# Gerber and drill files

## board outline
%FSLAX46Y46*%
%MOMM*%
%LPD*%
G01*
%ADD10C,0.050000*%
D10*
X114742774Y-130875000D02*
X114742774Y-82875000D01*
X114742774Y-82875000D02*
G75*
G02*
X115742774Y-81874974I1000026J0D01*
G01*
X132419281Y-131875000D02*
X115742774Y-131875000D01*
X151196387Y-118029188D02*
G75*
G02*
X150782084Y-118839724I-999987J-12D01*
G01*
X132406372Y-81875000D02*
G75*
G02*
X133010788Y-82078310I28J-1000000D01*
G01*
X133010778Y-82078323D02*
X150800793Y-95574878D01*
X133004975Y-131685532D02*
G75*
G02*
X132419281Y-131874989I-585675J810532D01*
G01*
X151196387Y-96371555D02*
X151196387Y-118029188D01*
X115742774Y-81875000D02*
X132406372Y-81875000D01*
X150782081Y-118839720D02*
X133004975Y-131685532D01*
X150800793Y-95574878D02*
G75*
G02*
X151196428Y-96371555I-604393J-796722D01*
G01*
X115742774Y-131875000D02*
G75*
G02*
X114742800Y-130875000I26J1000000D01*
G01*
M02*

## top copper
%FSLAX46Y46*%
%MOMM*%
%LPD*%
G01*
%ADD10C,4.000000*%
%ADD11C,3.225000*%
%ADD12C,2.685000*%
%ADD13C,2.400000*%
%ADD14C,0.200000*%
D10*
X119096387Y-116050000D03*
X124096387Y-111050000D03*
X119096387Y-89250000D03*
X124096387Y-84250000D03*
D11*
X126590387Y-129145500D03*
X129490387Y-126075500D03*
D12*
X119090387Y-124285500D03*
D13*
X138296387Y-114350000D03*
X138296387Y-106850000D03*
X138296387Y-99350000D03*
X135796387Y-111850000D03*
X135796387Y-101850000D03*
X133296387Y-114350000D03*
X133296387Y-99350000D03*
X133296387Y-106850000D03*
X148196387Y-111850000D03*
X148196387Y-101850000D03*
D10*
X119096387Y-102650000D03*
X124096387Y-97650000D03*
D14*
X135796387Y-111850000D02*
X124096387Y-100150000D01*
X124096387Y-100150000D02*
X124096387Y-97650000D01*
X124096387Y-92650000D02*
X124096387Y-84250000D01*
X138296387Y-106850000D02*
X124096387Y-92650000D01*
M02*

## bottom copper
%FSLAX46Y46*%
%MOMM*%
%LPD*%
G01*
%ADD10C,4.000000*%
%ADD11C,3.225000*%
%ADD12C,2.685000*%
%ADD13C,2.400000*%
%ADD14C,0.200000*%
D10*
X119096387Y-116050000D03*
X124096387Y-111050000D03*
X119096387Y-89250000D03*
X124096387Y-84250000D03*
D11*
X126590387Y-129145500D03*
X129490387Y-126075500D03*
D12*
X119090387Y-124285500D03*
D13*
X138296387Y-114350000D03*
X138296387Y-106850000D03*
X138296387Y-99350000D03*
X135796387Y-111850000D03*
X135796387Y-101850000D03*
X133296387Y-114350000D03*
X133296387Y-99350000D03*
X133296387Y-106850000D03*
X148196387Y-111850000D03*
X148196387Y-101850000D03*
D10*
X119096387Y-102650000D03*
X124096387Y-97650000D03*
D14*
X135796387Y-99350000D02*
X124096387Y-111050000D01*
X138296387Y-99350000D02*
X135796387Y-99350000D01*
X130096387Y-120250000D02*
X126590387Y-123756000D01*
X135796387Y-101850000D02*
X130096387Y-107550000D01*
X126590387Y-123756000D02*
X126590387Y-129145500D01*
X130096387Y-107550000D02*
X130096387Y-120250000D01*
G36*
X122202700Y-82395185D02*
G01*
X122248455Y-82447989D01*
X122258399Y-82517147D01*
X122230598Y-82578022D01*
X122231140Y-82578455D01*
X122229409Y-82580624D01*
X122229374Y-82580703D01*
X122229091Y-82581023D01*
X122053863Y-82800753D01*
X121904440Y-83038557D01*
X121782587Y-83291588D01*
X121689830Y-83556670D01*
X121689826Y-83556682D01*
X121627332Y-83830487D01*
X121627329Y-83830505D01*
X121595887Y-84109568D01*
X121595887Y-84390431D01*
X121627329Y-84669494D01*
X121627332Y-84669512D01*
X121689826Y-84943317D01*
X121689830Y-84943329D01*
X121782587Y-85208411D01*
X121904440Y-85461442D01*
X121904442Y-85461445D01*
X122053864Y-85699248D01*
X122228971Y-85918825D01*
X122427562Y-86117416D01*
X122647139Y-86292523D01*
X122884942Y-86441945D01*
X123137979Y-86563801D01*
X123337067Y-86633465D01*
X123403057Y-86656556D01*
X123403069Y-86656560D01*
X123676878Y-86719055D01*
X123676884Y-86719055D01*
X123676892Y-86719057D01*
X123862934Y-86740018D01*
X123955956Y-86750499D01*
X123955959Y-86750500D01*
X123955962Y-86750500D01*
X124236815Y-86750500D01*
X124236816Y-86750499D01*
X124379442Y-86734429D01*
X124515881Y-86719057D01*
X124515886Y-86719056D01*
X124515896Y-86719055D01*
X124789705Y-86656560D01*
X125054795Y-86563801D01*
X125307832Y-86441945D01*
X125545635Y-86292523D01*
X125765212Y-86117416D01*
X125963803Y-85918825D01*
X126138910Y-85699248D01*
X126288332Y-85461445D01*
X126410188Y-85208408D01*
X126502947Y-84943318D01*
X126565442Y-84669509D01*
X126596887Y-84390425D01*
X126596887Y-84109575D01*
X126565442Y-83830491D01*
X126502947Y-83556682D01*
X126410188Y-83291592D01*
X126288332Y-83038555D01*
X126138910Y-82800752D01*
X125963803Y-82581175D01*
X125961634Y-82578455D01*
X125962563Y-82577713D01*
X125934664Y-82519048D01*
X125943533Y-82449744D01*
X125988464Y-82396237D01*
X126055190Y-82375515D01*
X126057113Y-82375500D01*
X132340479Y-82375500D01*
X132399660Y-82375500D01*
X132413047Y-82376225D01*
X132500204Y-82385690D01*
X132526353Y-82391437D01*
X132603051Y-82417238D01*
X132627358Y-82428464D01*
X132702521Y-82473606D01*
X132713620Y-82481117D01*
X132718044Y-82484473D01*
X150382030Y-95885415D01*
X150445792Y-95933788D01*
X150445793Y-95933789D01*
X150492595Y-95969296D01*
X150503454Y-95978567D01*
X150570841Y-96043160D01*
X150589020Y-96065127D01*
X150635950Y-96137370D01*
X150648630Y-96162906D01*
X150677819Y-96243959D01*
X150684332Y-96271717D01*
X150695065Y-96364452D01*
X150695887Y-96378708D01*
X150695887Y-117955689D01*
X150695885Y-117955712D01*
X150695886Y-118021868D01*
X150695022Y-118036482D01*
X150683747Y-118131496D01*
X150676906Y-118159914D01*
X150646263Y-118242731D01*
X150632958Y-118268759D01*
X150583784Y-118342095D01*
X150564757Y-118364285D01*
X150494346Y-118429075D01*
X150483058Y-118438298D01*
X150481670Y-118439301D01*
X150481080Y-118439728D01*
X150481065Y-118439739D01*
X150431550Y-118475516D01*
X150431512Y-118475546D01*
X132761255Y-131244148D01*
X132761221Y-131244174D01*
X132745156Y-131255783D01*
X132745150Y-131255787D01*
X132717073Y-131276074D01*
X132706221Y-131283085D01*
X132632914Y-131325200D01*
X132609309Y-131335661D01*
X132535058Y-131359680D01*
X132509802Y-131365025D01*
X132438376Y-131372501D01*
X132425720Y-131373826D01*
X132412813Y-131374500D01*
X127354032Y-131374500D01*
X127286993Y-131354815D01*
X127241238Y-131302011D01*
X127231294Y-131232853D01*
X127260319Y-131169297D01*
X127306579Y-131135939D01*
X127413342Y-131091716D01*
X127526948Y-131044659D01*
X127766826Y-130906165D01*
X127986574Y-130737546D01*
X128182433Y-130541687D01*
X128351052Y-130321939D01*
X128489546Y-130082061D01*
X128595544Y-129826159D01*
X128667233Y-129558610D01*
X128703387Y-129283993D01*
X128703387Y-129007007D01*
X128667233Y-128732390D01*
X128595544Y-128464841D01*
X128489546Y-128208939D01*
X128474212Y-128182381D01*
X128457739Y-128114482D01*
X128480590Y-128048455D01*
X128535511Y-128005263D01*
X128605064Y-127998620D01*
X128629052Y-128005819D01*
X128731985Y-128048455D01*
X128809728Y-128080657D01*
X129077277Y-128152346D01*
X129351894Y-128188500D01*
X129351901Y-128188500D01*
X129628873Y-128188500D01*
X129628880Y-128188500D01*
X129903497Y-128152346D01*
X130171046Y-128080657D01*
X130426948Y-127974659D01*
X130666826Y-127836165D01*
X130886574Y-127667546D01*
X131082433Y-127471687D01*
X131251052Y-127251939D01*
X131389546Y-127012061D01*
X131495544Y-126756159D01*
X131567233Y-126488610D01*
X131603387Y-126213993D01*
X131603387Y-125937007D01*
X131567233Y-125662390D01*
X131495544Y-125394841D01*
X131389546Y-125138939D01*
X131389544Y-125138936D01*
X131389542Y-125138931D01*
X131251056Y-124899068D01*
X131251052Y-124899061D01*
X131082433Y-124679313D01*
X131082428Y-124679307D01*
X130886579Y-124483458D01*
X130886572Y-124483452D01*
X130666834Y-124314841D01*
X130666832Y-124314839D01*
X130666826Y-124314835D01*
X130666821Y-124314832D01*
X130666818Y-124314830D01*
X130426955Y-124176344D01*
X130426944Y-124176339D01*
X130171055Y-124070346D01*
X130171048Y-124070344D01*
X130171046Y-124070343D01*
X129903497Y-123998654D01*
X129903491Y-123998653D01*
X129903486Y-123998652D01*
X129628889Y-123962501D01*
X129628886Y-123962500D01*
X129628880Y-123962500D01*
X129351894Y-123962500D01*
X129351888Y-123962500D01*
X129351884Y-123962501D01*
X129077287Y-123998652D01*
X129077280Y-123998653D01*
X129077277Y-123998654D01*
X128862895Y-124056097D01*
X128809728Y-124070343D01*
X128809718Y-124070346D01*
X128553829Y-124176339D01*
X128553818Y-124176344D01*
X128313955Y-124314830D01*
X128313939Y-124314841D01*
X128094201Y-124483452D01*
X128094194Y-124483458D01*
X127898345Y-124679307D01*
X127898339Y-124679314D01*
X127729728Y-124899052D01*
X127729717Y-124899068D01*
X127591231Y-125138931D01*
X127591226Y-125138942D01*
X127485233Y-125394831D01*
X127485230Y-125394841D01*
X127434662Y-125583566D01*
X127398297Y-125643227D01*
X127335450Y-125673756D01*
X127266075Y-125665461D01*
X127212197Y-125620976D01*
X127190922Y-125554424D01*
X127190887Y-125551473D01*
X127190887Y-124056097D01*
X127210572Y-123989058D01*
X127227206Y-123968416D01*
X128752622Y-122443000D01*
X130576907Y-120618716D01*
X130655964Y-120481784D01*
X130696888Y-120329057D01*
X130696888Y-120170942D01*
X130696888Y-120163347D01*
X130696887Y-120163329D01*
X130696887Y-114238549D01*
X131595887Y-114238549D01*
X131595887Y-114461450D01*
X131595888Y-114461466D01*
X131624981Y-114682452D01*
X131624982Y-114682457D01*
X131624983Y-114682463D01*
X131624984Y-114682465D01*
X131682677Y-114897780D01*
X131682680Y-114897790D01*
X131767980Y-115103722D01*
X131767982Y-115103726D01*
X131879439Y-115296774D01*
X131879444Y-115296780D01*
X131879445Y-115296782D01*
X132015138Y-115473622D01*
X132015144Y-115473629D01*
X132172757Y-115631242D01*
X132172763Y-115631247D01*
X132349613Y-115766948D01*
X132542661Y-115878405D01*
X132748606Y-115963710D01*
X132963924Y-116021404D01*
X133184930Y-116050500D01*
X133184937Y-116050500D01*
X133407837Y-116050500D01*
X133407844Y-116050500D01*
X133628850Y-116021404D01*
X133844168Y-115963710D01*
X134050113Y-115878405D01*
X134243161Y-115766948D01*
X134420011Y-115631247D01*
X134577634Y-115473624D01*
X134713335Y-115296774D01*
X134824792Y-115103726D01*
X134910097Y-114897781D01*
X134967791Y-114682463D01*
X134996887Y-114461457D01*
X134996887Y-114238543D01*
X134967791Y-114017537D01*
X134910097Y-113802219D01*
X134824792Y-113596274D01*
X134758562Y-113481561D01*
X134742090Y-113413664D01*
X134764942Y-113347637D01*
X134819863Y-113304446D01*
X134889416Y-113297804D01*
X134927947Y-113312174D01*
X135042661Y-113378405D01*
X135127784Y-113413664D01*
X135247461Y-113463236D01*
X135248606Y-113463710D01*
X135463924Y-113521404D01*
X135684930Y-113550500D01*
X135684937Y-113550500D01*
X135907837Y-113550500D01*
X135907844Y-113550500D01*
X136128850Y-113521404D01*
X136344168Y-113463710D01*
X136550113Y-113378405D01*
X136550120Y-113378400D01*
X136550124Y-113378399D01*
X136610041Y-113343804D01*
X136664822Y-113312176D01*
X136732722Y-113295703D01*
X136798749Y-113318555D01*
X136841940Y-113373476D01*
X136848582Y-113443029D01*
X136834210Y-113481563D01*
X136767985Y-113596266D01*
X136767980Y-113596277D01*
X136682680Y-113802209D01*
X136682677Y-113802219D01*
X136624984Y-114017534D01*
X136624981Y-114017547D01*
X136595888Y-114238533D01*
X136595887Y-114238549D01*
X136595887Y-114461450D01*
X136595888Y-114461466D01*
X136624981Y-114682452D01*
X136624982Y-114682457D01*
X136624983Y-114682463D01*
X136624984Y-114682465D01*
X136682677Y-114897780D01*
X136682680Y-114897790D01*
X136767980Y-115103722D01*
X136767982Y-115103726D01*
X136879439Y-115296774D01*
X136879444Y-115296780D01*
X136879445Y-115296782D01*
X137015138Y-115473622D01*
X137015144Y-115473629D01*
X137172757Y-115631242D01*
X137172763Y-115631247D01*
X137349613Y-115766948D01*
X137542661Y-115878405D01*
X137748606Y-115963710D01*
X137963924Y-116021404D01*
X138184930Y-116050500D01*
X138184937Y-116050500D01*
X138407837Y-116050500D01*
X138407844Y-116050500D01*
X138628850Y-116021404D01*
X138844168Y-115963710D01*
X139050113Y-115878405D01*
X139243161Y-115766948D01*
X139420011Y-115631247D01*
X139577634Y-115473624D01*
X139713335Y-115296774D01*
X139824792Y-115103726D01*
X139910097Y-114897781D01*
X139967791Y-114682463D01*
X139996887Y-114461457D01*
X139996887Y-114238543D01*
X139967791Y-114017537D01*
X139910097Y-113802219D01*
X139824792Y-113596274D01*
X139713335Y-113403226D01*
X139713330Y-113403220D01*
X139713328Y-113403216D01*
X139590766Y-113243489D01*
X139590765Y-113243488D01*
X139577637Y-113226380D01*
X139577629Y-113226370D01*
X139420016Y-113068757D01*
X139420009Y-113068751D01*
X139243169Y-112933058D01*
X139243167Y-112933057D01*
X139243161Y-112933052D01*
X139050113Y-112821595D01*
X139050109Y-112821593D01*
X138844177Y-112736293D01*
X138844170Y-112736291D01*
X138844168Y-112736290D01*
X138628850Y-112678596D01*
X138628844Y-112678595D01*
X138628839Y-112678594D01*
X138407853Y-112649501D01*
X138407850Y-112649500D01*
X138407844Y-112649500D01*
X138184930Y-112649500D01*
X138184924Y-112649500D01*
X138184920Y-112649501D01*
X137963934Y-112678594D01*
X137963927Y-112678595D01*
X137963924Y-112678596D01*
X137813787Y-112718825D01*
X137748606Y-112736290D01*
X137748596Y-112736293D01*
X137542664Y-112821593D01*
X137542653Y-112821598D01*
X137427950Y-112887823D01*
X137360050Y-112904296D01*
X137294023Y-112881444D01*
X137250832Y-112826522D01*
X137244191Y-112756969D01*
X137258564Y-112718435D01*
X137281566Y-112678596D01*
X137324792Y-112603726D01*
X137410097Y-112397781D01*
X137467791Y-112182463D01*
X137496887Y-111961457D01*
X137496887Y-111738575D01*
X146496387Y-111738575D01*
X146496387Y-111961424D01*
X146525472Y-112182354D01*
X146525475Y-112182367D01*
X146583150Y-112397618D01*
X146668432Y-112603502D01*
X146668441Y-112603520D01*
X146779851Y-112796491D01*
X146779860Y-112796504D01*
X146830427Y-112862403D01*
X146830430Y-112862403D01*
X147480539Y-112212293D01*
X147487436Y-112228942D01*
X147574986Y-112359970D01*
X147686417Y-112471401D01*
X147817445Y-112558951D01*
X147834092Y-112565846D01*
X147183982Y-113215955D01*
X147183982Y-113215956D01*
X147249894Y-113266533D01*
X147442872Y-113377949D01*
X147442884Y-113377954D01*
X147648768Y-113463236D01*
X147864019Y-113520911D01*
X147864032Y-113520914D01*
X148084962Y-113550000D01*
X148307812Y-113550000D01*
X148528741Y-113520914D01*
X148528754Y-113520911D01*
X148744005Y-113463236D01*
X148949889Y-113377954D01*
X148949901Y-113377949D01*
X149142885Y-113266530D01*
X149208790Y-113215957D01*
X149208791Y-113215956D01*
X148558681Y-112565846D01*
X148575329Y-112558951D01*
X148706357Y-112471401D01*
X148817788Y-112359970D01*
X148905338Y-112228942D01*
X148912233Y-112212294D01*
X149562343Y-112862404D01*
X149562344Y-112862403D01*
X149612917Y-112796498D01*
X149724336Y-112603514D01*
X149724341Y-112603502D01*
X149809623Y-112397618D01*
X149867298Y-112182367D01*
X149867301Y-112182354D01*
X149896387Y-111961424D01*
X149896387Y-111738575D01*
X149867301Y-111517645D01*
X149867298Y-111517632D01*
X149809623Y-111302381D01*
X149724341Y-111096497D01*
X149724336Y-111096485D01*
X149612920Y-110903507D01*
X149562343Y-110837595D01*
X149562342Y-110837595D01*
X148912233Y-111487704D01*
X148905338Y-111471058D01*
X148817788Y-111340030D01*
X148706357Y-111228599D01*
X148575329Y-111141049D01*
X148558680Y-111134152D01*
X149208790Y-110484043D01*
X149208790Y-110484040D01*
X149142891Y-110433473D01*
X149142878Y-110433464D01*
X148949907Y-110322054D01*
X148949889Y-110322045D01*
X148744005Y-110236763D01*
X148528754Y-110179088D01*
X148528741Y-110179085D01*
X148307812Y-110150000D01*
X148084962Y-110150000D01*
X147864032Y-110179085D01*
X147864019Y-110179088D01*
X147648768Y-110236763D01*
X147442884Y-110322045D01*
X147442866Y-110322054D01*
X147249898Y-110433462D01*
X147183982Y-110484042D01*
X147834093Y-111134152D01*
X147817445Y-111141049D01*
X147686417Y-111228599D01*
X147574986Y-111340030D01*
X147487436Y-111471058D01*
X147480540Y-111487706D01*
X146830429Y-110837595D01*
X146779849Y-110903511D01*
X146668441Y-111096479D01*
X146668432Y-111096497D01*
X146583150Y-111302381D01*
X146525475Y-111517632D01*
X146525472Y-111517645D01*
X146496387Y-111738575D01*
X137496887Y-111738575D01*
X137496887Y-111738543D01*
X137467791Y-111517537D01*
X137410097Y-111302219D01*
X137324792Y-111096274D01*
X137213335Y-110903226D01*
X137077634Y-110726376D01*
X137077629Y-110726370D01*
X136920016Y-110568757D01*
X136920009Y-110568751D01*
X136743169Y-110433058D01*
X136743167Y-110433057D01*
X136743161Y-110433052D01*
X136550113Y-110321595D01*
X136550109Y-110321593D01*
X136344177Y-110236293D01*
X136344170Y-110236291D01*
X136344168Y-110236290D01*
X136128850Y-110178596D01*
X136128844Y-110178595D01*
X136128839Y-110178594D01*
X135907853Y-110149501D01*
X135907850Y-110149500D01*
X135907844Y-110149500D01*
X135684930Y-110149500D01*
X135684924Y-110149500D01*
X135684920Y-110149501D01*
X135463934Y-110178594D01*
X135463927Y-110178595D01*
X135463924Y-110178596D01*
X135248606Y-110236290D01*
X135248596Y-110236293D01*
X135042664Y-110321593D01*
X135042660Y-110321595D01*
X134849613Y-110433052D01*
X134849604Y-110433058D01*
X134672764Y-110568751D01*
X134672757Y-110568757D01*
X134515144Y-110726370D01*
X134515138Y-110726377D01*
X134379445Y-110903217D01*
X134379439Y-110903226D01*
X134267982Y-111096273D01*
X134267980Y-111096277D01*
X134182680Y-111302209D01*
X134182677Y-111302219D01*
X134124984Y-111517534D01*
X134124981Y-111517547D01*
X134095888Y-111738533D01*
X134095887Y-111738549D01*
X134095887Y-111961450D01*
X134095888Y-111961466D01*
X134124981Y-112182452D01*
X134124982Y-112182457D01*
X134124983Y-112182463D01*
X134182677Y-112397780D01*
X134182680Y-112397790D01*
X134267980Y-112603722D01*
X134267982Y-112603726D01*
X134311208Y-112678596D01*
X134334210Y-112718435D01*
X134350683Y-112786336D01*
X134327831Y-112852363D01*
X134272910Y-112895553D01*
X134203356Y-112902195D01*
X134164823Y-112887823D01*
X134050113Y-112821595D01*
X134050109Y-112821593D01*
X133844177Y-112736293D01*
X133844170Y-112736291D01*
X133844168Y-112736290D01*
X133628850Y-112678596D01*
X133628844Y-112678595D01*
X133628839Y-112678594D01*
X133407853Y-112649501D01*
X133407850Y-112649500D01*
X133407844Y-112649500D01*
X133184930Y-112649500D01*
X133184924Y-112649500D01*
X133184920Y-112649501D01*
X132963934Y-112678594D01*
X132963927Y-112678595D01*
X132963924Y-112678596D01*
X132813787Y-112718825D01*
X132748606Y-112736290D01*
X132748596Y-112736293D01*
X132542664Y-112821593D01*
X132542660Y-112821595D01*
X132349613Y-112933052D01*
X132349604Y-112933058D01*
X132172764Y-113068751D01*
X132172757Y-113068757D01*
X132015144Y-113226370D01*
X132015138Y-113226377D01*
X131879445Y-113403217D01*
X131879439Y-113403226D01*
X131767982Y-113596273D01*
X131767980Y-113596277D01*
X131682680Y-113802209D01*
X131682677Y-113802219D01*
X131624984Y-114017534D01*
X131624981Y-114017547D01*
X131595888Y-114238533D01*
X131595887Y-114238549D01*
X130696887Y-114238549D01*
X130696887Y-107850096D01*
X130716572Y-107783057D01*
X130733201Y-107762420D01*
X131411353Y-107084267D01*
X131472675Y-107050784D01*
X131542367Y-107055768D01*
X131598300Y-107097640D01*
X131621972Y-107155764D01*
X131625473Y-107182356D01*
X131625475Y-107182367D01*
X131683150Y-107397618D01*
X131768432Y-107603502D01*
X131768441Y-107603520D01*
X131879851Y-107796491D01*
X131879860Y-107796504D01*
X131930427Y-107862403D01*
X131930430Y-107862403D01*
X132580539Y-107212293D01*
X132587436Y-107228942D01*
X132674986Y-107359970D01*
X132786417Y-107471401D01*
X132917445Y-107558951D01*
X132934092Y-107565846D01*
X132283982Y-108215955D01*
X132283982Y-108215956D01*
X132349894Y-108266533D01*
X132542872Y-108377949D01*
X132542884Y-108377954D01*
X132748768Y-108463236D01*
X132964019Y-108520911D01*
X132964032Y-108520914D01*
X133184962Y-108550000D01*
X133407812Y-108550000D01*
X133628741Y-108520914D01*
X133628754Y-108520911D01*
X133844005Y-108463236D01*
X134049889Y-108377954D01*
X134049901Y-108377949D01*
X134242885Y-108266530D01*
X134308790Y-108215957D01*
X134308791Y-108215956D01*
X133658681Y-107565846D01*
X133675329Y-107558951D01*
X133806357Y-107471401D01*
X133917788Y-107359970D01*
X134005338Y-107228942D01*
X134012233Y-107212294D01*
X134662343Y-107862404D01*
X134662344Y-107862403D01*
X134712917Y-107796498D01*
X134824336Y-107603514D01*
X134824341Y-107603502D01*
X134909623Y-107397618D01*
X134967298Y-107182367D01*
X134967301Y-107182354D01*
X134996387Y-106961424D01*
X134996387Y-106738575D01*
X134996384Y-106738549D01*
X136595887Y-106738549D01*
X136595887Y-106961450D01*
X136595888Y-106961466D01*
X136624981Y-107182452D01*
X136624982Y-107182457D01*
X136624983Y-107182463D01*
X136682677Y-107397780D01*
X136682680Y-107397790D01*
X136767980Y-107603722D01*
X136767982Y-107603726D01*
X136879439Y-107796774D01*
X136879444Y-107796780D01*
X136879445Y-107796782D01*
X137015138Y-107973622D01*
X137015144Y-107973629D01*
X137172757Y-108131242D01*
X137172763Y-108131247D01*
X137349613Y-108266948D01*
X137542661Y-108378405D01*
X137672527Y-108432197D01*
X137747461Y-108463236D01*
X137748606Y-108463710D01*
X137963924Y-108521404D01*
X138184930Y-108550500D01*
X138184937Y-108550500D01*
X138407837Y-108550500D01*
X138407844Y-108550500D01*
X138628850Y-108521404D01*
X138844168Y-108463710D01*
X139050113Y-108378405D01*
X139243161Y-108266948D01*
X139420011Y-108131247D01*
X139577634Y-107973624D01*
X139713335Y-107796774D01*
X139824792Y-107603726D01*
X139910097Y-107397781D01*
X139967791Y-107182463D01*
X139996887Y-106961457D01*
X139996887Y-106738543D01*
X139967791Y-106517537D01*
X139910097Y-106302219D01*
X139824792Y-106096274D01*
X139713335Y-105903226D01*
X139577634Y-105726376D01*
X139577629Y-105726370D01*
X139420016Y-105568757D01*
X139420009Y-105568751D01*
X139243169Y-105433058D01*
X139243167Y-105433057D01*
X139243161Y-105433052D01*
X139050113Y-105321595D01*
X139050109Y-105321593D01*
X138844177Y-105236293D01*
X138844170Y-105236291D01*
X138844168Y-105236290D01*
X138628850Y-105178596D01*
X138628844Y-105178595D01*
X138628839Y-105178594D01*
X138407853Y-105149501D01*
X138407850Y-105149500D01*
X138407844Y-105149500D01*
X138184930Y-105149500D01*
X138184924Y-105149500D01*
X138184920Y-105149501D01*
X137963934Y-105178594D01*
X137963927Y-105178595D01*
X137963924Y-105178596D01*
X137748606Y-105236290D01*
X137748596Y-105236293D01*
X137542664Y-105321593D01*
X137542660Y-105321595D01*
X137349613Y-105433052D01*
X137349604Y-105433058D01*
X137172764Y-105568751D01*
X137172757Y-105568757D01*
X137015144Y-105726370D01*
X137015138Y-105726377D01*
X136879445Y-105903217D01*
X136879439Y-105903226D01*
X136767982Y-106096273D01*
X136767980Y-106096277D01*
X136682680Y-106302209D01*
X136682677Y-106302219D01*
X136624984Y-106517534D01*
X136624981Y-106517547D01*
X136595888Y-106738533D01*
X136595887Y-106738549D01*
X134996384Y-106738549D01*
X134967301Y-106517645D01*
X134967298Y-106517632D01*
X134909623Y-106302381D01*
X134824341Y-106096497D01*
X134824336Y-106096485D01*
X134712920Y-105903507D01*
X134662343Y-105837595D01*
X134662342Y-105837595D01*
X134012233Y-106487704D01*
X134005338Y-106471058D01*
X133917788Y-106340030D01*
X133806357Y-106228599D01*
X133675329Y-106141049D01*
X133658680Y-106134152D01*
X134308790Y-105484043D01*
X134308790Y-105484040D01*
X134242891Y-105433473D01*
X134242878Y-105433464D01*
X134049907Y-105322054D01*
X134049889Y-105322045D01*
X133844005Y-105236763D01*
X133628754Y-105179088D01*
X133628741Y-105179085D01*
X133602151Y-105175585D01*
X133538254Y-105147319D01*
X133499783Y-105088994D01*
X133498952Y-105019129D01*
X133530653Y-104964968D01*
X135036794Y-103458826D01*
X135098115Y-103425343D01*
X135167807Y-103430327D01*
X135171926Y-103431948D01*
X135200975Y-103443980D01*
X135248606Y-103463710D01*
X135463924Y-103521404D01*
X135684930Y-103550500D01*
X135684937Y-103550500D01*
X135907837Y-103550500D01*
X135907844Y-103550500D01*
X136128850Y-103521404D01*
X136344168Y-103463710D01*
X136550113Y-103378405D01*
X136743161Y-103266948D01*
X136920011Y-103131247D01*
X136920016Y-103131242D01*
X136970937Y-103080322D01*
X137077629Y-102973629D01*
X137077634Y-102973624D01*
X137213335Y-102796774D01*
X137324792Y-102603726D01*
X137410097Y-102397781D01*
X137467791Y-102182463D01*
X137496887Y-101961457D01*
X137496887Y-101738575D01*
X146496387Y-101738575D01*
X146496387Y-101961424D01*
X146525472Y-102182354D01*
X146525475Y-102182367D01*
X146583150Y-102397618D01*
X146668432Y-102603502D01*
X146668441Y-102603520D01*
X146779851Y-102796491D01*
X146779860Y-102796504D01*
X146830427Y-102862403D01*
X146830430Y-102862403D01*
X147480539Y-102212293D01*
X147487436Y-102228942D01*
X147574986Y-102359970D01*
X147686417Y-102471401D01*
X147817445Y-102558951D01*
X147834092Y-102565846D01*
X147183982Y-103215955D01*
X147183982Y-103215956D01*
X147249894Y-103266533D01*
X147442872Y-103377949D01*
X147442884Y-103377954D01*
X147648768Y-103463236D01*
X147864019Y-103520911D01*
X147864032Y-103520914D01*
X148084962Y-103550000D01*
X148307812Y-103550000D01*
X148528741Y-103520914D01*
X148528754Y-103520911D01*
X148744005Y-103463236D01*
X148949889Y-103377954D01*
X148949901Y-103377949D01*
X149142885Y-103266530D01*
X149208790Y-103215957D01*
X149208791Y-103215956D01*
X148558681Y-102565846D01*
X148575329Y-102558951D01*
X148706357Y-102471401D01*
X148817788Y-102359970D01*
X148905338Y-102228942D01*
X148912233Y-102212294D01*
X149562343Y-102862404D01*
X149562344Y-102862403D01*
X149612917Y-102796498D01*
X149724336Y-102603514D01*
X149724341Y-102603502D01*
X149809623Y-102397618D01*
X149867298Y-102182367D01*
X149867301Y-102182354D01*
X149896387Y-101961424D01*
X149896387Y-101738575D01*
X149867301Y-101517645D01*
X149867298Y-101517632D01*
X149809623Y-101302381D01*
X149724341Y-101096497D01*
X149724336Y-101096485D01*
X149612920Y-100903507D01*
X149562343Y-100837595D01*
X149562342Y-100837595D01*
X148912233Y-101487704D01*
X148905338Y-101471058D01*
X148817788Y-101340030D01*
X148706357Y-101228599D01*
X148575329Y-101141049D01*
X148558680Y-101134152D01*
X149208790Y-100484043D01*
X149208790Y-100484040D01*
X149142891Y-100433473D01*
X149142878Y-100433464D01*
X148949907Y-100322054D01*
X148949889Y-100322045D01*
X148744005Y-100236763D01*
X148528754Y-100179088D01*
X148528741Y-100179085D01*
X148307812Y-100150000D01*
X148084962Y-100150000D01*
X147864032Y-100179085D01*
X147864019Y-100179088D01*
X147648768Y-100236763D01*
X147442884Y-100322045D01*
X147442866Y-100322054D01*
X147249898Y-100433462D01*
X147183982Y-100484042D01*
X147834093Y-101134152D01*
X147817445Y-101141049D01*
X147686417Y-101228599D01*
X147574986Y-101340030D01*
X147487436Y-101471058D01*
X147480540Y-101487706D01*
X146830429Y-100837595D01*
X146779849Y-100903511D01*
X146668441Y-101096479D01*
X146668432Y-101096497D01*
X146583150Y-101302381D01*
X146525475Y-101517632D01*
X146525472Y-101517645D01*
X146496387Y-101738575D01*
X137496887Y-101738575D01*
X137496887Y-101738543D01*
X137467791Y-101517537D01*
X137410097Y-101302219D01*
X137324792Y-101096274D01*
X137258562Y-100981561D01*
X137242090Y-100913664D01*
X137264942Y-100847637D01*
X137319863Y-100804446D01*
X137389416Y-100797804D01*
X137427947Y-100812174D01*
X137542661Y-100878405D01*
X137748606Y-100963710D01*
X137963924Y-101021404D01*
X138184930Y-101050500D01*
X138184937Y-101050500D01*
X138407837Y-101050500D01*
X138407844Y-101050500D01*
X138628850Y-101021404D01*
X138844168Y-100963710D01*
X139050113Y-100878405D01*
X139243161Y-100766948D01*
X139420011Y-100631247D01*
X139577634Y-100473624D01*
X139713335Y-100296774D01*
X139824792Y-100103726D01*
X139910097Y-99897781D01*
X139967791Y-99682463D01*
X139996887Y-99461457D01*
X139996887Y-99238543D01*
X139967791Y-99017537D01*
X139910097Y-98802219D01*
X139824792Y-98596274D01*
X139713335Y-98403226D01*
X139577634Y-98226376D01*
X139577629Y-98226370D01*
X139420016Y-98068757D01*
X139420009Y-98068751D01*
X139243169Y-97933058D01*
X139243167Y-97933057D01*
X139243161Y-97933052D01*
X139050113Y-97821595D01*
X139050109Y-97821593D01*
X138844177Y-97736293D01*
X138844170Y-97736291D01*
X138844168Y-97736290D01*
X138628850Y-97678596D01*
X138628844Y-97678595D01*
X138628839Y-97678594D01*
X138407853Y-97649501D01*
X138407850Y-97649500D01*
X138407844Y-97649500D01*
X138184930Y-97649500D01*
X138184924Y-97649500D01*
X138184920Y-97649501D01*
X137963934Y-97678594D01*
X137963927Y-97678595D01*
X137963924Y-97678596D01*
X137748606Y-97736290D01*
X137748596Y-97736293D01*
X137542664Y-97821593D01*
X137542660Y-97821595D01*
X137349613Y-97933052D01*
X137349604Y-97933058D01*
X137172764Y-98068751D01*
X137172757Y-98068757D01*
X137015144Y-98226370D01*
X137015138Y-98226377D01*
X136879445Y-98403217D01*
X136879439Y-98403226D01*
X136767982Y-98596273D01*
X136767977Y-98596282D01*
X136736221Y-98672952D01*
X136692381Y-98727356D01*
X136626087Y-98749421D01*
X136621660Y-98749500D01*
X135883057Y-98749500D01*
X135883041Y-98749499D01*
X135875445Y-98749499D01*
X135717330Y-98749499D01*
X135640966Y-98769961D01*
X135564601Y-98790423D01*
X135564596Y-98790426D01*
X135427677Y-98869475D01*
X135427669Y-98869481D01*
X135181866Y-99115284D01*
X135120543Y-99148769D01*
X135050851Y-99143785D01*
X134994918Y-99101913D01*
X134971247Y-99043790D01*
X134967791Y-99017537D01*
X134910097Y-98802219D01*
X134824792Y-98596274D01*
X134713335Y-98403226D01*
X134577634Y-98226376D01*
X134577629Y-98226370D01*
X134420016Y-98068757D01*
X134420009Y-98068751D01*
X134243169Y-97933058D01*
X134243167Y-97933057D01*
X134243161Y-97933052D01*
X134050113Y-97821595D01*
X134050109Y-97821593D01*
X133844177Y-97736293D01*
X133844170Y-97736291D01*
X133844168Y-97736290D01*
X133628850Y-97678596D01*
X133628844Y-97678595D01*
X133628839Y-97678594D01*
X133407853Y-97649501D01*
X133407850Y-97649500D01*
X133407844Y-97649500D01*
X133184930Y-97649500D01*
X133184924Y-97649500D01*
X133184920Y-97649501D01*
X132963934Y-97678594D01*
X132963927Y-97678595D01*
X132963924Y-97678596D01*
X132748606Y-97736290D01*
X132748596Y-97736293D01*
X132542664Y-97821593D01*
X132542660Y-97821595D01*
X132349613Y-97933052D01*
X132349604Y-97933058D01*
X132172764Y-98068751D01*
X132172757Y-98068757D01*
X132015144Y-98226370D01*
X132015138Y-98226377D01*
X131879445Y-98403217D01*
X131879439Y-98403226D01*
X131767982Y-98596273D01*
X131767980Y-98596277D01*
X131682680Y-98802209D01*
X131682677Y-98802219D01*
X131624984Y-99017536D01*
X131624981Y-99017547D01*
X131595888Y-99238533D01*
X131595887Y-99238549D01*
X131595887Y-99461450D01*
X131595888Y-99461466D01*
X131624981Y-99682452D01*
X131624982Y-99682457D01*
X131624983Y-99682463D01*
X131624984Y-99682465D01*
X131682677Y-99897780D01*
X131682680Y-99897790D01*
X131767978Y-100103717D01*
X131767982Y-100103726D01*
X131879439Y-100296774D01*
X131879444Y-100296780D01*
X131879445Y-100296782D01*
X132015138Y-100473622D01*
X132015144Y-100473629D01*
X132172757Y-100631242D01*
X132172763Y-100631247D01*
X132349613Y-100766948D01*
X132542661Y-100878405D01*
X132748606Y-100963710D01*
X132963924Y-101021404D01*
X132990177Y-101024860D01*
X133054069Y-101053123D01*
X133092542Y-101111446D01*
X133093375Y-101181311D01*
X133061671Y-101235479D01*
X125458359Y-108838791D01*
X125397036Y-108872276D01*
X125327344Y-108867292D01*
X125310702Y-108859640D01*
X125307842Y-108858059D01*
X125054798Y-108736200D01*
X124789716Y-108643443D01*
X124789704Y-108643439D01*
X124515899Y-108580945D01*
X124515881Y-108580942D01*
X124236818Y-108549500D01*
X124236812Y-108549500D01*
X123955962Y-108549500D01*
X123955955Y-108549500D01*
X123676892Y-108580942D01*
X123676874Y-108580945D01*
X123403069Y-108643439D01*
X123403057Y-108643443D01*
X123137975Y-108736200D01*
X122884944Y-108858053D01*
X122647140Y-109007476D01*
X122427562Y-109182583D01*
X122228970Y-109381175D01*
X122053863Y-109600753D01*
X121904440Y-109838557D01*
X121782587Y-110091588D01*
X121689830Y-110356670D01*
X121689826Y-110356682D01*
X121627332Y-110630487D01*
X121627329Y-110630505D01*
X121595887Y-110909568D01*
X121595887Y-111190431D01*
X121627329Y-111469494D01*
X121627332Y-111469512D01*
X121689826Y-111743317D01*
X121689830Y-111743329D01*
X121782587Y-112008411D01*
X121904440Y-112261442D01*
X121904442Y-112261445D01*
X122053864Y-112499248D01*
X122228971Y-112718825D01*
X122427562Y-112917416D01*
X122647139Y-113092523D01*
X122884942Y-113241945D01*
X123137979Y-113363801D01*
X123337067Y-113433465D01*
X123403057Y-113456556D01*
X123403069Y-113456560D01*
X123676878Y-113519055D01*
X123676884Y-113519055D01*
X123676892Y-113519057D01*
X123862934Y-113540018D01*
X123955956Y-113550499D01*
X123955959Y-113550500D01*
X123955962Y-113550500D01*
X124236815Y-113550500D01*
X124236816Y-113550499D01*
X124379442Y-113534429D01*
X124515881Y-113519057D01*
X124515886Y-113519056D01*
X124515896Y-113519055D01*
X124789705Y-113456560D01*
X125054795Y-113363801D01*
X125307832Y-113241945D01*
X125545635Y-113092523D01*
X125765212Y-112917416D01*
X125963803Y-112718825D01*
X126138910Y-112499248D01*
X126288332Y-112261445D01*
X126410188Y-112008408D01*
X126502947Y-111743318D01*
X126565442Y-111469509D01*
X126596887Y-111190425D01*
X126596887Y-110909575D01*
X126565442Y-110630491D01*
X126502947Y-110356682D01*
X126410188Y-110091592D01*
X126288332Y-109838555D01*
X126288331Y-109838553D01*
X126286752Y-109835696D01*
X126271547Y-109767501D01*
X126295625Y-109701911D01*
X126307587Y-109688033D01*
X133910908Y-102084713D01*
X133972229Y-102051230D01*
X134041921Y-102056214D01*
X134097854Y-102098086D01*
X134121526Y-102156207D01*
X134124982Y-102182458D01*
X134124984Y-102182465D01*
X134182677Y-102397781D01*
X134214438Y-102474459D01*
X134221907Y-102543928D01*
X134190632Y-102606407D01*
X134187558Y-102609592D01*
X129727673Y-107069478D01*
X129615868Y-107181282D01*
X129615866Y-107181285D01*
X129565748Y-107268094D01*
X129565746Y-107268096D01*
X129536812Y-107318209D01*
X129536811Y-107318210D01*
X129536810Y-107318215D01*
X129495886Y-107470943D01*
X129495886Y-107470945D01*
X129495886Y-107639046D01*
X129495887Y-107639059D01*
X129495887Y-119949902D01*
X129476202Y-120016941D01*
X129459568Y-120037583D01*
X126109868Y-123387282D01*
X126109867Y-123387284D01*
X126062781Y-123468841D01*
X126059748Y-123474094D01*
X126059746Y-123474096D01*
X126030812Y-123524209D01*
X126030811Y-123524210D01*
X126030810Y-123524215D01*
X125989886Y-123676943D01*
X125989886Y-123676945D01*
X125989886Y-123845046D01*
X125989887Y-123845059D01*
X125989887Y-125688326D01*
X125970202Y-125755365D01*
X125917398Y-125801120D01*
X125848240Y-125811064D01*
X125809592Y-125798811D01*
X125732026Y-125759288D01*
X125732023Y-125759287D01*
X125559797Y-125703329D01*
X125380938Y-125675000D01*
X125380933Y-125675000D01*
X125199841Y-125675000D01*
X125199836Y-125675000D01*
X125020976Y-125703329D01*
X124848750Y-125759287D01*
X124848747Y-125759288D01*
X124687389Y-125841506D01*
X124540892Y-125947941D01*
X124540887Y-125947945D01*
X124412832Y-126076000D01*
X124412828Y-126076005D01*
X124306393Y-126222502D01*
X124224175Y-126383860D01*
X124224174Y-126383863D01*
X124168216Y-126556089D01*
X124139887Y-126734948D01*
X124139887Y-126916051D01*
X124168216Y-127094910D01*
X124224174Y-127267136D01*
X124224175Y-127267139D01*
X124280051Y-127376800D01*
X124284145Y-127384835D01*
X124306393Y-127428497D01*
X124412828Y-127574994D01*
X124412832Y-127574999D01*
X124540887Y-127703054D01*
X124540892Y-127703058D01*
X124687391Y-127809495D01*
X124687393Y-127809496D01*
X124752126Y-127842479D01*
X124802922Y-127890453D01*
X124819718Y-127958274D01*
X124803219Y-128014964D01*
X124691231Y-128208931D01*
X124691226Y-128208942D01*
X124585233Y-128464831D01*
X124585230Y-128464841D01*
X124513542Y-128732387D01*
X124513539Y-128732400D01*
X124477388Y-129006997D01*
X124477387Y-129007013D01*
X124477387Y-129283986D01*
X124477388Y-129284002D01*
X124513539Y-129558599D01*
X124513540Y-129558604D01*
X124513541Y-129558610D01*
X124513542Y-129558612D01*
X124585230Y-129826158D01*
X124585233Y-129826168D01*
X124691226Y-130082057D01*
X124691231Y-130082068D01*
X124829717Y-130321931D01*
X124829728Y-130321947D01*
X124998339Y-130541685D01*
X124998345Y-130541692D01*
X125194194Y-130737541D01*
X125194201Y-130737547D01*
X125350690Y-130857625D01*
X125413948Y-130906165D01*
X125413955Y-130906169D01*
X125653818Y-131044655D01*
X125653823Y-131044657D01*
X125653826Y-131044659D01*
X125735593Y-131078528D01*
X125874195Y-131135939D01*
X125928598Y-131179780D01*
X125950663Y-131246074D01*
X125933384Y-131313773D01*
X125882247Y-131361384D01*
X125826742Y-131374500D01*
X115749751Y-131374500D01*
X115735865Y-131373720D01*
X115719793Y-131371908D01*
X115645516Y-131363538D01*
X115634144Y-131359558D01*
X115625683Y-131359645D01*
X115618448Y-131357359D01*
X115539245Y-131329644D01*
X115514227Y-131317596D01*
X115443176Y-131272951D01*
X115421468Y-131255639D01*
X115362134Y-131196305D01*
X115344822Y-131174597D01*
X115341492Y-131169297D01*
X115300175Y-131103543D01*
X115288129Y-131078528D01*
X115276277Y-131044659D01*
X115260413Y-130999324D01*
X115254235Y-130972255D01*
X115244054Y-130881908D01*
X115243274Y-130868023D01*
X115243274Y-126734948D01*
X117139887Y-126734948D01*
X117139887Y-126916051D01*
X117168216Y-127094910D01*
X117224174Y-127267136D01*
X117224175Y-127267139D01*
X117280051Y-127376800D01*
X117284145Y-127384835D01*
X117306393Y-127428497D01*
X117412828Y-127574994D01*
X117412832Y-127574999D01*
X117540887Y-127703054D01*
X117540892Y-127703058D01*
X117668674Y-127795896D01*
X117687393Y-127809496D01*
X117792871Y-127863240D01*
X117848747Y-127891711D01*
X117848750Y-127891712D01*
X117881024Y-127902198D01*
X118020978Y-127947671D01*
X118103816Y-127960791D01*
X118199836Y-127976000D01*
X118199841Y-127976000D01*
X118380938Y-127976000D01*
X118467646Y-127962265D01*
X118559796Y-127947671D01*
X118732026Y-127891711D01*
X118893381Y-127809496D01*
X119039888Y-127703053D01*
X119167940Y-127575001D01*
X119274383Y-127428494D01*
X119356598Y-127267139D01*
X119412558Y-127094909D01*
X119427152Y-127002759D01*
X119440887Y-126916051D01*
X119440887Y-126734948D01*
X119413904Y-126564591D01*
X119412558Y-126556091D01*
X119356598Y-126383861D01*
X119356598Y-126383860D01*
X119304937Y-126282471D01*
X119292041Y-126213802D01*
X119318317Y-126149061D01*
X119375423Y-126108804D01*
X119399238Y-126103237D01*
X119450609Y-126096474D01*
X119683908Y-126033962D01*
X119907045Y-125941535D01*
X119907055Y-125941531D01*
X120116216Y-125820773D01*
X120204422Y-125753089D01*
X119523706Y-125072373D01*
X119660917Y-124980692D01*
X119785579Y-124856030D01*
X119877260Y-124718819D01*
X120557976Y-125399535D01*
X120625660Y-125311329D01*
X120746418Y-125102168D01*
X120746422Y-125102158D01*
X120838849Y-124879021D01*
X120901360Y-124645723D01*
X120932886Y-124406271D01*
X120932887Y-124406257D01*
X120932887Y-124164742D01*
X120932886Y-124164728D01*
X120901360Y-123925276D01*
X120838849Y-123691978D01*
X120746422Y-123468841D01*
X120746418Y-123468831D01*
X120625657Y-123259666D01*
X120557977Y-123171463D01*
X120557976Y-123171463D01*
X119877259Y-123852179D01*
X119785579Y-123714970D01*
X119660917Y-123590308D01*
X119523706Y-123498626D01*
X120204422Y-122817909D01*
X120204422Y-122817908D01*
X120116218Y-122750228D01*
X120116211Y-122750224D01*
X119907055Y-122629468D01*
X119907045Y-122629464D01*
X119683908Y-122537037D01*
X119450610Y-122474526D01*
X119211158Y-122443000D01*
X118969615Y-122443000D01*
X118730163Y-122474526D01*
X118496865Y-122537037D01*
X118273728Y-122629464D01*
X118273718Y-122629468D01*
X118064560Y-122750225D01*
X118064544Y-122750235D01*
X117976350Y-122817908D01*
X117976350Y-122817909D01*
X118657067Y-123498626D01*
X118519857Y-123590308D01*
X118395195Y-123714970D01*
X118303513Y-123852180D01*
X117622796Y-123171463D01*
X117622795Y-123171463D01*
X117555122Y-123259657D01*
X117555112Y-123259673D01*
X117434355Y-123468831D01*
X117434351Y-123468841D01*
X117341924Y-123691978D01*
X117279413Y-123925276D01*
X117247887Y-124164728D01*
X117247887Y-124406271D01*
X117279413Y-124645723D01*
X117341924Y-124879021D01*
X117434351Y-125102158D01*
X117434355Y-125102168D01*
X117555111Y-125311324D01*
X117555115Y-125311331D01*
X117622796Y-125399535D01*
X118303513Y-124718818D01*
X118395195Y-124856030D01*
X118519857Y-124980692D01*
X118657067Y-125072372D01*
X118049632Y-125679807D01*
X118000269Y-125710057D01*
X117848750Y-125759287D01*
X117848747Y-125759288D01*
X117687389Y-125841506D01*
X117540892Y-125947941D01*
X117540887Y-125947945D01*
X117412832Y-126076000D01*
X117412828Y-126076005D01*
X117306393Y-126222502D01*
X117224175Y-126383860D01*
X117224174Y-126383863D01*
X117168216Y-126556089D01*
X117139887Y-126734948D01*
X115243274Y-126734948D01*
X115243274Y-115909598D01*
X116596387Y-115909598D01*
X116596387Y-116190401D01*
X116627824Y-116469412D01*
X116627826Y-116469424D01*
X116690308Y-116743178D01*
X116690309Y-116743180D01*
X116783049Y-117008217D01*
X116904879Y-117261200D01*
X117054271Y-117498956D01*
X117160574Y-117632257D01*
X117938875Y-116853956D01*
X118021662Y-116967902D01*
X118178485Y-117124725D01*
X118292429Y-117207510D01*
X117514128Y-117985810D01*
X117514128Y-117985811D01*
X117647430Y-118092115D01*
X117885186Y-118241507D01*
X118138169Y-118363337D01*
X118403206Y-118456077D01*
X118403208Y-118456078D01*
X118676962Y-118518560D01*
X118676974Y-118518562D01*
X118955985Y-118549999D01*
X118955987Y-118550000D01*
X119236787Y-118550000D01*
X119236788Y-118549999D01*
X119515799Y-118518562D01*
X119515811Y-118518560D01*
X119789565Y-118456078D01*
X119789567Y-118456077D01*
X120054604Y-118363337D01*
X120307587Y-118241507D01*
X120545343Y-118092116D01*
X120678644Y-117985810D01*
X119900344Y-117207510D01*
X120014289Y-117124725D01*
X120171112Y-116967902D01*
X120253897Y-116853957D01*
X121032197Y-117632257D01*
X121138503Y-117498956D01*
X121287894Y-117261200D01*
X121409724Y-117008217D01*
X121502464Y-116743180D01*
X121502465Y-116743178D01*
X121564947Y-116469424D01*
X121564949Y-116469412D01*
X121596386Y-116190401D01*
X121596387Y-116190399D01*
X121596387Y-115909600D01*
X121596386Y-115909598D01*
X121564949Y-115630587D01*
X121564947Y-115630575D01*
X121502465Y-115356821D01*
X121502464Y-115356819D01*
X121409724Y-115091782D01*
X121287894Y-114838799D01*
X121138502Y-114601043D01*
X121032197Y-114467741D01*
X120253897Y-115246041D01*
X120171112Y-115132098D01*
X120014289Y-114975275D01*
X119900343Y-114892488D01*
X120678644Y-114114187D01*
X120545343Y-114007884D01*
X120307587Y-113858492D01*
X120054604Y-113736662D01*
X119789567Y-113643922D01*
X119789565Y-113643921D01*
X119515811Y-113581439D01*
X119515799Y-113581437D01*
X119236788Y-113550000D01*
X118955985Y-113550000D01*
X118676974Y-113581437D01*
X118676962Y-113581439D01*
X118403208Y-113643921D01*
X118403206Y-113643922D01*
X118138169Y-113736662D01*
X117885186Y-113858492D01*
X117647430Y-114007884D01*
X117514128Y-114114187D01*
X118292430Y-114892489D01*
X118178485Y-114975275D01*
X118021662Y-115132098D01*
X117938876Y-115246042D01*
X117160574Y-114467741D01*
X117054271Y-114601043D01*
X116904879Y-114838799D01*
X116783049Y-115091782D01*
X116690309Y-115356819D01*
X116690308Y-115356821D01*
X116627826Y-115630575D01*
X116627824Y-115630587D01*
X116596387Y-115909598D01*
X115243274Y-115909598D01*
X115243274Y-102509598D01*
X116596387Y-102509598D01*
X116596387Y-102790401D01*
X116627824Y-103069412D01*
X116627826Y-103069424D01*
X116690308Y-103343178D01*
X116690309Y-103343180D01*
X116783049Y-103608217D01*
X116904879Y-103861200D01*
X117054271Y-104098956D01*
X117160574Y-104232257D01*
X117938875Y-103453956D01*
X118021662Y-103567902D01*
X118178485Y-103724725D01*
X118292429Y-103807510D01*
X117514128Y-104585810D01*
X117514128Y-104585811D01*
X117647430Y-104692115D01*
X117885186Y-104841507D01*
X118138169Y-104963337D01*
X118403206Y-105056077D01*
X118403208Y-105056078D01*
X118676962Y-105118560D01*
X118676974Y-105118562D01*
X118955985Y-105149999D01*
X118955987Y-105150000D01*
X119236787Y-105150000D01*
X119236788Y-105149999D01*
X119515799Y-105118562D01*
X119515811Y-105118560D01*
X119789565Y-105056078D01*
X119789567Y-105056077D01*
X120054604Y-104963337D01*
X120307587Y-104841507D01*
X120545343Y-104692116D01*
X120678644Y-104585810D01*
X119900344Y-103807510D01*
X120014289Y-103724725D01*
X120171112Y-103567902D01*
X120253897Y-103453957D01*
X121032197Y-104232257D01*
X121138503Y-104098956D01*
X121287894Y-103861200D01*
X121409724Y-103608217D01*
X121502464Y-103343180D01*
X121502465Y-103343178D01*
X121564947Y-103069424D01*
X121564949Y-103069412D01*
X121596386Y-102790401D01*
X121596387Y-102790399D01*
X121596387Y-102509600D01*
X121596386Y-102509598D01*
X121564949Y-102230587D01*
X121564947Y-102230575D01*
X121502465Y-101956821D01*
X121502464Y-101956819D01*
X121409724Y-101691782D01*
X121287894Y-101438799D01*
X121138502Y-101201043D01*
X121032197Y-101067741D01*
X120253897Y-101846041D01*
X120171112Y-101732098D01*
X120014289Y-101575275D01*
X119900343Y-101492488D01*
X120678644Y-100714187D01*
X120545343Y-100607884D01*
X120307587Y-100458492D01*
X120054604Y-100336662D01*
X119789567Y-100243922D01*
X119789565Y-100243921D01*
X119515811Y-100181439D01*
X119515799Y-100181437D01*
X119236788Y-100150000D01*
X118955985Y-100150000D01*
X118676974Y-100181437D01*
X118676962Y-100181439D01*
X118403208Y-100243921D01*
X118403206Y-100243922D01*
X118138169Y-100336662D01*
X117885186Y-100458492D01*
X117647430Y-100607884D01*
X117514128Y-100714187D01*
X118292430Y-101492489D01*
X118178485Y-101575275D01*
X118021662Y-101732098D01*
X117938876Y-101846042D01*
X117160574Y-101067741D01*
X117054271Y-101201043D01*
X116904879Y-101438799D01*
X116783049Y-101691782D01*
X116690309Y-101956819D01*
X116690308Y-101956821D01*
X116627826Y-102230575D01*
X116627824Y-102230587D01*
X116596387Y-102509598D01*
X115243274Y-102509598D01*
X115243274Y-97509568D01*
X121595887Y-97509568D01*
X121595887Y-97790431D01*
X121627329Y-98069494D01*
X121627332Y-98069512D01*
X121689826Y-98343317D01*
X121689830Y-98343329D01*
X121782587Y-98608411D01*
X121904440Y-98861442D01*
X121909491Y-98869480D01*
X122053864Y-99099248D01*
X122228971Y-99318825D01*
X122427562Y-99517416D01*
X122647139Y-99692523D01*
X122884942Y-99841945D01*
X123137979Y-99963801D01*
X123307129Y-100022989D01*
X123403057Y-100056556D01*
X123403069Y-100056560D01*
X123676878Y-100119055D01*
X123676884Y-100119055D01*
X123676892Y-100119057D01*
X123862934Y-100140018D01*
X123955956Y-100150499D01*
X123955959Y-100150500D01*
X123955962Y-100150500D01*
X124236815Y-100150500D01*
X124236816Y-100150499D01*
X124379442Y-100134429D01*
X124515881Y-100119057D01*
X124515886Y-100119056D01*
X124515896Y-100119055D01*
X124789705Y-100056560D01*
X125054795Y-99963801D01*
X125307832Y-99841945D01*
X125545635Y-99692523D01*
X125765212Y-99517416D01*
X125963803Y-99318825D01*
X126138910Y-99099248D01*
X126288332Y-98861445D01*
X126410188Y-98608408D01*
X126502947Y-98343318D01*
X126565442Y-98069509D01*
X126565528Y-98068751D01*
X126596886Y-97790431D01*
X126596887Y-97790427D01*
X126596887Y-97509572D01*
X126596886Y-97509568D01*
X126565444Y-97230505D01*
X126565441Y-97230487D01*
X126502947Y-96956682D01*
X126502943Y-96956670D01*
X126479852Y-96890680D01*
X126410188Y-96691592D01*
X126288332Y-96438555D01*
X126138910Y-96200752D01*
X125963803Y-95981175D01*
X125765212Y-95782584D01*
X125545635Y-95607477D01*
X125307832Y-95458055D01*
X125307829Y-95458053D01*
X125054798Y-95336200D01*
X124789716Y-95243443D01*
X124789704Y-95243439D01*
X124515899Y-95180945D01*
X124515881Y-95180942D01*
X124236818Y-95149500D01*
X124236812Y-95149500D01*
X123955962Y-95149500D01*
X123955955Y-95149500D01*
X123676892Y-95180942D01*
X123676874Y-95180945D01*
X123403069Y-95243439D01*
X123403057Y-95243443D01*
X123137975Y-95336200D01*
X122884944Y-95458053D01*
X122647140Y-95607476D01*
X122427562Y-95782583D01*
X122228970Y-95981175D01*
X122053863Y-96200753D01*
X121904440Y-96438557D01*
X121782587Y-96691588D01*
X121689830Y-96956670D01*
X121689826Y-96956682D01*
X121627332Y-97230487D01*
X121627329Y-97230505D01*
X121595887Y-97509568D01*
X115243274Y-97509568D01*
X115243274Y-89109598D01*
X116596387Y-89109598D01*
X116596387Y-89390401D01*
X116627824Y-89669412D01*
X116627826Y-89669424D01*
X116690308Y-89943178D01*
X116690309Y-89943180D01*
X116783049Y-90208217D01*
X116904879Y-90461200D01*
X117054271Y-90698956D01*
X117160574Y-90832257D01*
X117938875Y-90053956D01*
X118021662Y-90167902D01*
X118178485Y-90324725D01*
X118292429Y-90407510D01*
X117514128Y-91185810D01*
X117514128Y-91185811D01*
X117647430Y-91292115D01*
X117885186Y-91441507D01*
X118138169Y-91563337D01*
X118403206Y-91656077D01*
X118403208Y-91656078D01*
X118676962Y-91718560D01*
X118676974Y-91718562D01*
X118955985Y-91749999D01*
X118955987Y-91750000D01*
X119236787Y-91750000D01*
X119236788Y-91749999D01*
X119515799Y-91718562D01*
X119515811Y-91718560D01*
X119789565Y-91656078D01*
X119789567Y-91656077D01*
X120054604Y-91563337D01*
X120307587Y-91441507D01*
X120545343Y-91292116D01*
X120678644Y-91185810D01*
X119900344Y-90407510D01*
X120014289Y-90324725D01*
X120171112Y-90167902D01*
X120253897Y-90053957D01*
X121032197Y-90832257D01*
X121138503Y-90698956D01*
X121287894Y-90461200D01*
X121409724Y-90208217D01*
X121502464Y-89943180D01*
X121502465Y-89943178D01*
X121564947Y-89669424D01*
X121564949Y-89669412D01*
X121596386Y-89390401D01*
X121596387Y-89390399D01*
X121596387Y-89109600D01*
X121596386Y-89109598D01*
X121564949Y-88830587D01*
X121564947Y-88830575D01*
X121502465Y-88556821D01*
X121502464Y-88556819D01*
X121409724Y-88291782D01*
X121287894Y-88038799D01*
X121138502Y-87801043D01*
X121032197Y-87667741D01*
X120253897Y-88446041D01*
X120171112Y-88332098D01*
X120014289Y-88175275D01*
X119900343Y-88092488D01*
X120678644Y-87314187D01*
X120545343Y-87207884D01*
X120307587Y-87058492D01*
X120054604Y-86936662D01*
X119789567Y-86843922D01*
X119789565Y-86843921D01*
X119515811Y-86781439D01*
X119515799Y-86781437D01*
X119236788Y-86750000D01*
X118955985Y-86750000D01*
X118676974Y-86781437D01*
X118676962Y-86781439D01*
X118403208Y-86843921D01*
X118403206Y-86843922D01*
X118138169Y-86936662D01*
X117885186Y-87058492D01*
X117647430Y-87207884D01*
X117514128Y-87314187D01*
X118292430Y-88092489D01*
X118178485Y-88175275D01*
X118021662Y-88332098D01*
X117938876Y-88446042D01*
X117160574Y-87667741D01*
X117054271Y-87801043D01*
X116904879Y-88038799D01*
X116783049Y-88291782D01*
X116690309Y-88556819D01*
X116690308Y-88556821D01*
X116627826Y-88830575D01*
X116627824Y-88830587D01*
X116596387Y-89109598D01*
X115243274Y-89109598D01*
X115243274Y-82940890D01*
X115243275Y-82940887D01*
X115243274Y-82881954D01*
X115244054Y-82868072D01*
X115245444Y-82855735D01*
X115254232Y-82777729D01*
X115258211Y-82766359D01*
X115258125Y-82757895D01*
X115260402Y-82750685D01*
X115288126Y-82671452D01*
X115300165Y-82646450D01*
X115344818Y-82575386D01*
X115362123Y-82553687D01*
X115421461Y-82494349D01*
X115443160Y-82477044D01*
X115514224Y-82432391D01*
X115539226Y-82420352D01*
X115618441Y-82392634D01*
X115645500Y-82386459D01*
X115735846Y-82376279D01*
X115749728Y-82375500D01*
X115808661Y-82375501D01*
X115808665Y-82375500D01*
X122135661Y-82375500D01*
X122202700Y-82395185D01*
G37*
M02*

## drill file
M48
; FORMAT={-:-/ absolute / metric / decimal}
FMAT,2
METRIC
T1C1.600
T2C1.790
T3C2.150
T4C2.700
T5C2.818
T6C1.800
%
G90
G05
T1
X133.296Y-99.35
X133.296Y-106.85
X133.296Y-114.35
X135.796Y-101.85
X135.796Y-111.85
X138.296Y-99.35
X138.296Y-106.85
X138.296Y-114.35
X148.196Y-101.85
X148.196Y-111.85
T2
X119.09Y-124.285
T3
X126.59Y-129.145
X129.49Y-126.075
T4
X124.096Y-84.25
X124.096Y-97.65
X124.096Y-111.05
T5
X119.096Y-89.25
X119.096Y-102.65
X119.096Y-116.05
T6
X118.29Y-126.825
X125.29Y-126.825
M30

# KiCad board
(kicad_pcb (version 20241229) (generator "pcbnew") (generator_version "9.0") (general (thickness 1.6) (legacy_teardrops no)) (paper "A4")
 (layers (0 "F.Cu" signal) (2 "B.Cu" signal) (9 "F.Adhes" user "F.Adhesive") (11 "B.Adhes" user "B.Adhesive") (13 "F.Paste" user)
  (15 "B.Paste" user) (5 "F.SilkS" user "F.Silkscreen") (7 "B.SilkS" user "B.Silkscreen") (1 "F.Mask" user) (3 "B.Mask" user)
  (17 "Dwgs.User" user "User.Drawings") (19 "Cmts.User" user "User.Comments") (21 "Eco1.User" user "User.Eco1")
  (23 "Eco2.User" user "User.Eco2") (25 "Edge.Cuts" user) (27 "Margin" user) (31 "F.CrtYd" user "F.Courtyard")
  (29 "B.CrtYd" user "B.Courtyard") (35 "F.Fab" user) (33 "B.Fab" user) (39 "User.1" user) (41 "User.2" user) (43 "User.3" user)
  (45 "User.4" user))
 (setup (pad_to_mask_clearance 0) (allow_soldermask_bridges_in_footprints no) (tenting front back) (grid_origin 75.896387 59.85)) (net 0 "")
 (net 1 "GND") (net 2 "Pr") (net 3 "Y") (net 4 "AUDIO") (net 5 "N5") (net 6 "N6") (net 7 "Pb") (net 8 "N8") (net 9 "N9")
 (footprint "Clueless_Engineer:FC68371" (layer "F.Cu") (at 119.096387 116.05)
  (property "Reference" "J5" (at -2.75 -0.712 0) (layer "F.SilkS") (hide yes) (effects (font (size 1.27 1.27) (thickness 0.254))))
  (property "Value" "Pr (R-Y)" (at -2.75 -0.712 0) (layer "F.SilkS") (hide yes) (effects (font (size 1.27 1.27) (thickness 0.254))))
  (pad "1" thru_hole circle (at 0 0) (size 4 4) (drill 2.818) (layers "*.Cu" "*.Mask") (remove_unused_layers no) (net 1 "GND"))
  (pad "3" thru_hole circle (at 5 -5) (size 4 4) (drill 2.7) (layers "*.Cu" "*.Mask") (remove_unused_layers no) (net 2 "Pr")))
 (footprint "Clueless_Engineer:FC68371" (layer "F.Cu") (at 119.096387 89.25)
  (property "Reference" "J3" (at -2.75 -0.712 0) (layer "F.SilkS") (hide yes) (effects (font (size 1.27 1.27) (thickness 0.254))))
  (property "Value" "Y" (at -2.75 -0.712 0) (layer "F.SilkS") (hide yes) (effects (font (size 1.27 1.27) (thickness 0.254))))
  (pad "1" thru_hole circle (at 0 0) (size 4 4) (drill 2.818) (layers "*.Cu" "*.Mask") (remove_unused_layers no) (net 1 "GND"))
  (pad "3" thru_hole circle (at 5 -5) (size 4 4) (drill 2.7) (layers "*.Cu" "*.Mask") (remove_unused_layers no) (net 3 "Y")))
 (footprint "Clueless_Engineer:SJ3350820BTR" (layer "F.Cu") (at 126.590387 129.1455)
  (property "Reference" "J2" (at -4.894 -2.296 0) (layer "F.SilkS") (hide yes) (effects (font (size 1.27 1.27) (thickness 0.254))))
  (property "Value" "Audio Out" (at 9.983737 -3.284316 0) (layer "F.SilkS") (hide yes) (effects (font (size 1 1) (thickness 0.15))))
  (pad "" np_thru_hole circle (at -8.3 -2.32) (size 1.8 1.8) (drill 1.8) (layers "*.Cu" "*.Mask"))
  (pad "" np_thru_hole circle (at -1.3 -2.32) (size 1.8 1.8) (drill 1.8) (layers "*.Cu" "*.Mask"))
  (pad "2" thru_hole circle (at 0 0) (size 3.225 3.225) (drill 2.15) (layers "*.Cu" "*.Mask") (remove_unused_layers no) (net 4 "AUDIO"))
  (pad "3" thru_hole circle (at 2.9 -3.07) (size 3.225 3.225) (drill 2.15) (layers "*.Cu" "*.Mask") (remove_unused_layers no) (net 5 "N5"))
  (pad "5" thru_hole circle (at -7.5 -4.86) (size 2.685 2.685) (drill 1.79) (layers "*.Cu" "*.Mask") (remove_unused_layers no) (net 1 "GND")))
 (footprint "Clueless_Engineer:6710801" (layer "F.Cu") (at 138.296387 114.35 -90)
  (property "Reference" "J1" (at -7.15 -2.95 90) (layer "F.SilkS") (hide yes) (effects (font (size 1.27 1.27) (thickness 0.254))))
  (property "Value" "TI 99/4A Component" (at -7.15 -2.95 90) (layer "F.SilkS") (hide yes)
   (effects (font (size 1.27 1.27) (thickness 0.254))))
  (pad "1" thru_hole circle (at 0 0 270) (size 2.4 2.4) (drill 1.6) (layers "*.Cu" "*.Mask") (remove_unused_layers no) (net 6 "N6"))
  (pad "2" thru_hole circle (at -7.5 0 270) (size 2.4 2.4) (drill 1.6) (layers "*.Cu" "*.Mask") (remove_unused_layers no) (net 3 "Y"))
  (pad "3" thru_hole circle (at -15 0 270) (size 2.4 2.4) (drill 1.6) (layers "*.Cu" "*.Mask") (remove_unused_layers no) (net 2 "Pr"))
  (pad "4" thru_hole circle (at -2.5 2.5 270) (size 2.4 2.4) (drill 1.6) (layers "*.Cu" "*.Mask") (remove_unused_layers no) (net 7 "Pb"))
  (pad "5" thru_hole circle (at -12.5 2.5 270) (size 2.4 2.4) (drill 1.6) (layers "*.Cu" "*.Mask") (remove_unused_layers no) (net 4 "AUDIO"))
  (pad "6" thru_hole circle (at 0 5 270) (size 2.4 2.4) (drill 1.6) (layers "*.Cu" "*.Mask") (remove_unused_layers no) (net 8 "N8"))
  (pad "7" thru_hole circle (at -15 5 270) (size 2.4 2.4) (drill 1.6) (layers "*.Cu" "*.Mask") (remove_unused_layers no) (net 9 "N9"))
  (pad "8" thru_hole circle (at -7.5 5 270) (size 2.4 2.4) (drill 1.6) (layers "*.Cu" "*.Mask") (remove_unused_layers no) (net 1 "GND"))
  (pad "MH1" thru_hole circle (at -2.5 -9.9 270) (size 2.4 2.4) (drill 1.6) (layers "*.Cu" "*.Mask") (remove_unused_layers no) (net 1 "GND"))
  (pad "MH2" thru_hole circle (at -12.5 -9.9 270) (size 2.4 2.4) (drill 1.6) (layers "*.Cu" "*.Mask") (remove_unused_layers no)
   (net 1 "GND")))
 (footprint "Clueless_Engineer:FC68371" (layer "F.Cu") (at 119.096387 102.65)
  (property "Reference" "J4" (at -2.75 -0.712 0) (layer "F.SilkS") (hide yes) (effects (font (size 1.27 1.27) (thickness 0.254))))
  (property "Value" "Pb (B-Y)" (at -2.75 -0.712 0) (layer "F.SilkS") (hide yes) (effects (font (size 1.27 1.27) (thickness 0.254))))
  (pad "1" thru_hole circle (at 0 0) (size 4 4) (drill 2.818) (layers "*.Cu" "*.Mask") (remove_unused_layers no) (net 1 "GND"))
  (pad "3" thru_hole circle (at 5 -5) (size 4 4) (drill 2.7) (layers "*.Cu" "*.Mask") (remove_unused_layers no) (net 7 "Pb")))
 (gr_line (start 114.742774 130.875) (end 114.742774 82.875) (stroke (width 0.05) (type default)) (layer "Edge.Cuts"))
 (gr_arc (start 114.742774 82.875) (mid 115.035666 82.167889) (end 115.742774 81.875) (stroke (width 0.05) (type default))
  (layer "Edge.Cuts"))
 (gr_line (start 132.419281 131.875) (end 115.742774 131.875) (stroke (width 0.05) (type default)) (layer "Edge.Cuts"))
 (gr_arc (start 151.196387 118.029188) (mid 151.086811 118.484332) (end 150.782081 118.83972) (stroke (width 0.05) (type default))
  (layer "Edge.Cuts"))
 (gr_arc (start 132.406372 81.875) (mid 132.725216 81.927193) (end 133.010778 82.078323) (stroke (width 0.05) (type default))
  (layer "Edge.Cuts"))
 (gr_line (start 133.010778 82.078323) (end 150.800793 95.574878) (stroke (width 0.05) (type default)) (layer "Edge.Cuts"))
 (gr_arc (start 133.004975 131.685532) (mid 132.72707 131.826455) (end 132.419281 131.875) (stroke (width 0.05) (type default))
  (layer "Edge.Cuts"))
 (gr_line (start 151.196387 96.371555) (end 151.196387 118.029188) (stroke (width 0.05) (type default)) (layer "Edge.Cuts"))
 (gr_line (start 115.742774 81.875) (end 132.406372 81.875) (stroke (width 0.05) (type default)) (layer "Edge.Cuts"))
 (gr_line (start 150.782081 118.83972) (end 133.004975 131.685532) (stroke (width 0.05) (type default)) (layer "Edge.Cuts"))
 (gr_arc (start 150.800793 95.574878) (mid 151.092045 95.926811) (end 151.196387 96.371555) (stroke (width 0.05) (type default))
  (layer "Edge.Cuts"))
 (gr_arc (start 115.742774 131.875) (mid 115.035676 131.582102) (end 114.742774 130.875) (stroke (width 0.05) (type default))
  (layer "Edge.Cuts"))
 (segment (start 135.796387 111.85) (end 124.096387 100.15) (width 0.2) (layer "F.Cu") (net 7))
 (segment (start 124.096387 100.15) (end 124.096387 97.65) (width 0.2) (layer "F.Cu") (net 7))
 (segment (start 135.796387 99.35) (end 124.096387 111.05) (width 0.2) (layer "B.Cu") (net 2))
 (segment (start 138.296387 99.35) (end 135.796387 99.35) (width 0.2) (layer "B.Cu") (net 2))
 (segment (start 130.096387 120.25) (end 126.590387 123.756) (width 0.2) (layer "B.Cu") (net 4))
 (segment (start 135.796387 101.85) (end 130.096387 107.55) (width 0.2) (layer "B.Cu") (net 4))
 (segment (start 126.590387 123.756) (end 126.590387 129.1455) (width 0.2) (layer "B.Cu") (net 4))
 (segment (start 130.096387 107.55) (end 130.096387 120.25) (width 0.2) (layer "B.Cu") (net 4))
 (segment (start 124.096387 92.65) (end 124.096387 84.25) (width 0.2) (layer "F.Cu") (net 3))
 (segment (start 138.296387 106.85) (end 124.096387 92.65) (width 0.2) (layer "F.Cu") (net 3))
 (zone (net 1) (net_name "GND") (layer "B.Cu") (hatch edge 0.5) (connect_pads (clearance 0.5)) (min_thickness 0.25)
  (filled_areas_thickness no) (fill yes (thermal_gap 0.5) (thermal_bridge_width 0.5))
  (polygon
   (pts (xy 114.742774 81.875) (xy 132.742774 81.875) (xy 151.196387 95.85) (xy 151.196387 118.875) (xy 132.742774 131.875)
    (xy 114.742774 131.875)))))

